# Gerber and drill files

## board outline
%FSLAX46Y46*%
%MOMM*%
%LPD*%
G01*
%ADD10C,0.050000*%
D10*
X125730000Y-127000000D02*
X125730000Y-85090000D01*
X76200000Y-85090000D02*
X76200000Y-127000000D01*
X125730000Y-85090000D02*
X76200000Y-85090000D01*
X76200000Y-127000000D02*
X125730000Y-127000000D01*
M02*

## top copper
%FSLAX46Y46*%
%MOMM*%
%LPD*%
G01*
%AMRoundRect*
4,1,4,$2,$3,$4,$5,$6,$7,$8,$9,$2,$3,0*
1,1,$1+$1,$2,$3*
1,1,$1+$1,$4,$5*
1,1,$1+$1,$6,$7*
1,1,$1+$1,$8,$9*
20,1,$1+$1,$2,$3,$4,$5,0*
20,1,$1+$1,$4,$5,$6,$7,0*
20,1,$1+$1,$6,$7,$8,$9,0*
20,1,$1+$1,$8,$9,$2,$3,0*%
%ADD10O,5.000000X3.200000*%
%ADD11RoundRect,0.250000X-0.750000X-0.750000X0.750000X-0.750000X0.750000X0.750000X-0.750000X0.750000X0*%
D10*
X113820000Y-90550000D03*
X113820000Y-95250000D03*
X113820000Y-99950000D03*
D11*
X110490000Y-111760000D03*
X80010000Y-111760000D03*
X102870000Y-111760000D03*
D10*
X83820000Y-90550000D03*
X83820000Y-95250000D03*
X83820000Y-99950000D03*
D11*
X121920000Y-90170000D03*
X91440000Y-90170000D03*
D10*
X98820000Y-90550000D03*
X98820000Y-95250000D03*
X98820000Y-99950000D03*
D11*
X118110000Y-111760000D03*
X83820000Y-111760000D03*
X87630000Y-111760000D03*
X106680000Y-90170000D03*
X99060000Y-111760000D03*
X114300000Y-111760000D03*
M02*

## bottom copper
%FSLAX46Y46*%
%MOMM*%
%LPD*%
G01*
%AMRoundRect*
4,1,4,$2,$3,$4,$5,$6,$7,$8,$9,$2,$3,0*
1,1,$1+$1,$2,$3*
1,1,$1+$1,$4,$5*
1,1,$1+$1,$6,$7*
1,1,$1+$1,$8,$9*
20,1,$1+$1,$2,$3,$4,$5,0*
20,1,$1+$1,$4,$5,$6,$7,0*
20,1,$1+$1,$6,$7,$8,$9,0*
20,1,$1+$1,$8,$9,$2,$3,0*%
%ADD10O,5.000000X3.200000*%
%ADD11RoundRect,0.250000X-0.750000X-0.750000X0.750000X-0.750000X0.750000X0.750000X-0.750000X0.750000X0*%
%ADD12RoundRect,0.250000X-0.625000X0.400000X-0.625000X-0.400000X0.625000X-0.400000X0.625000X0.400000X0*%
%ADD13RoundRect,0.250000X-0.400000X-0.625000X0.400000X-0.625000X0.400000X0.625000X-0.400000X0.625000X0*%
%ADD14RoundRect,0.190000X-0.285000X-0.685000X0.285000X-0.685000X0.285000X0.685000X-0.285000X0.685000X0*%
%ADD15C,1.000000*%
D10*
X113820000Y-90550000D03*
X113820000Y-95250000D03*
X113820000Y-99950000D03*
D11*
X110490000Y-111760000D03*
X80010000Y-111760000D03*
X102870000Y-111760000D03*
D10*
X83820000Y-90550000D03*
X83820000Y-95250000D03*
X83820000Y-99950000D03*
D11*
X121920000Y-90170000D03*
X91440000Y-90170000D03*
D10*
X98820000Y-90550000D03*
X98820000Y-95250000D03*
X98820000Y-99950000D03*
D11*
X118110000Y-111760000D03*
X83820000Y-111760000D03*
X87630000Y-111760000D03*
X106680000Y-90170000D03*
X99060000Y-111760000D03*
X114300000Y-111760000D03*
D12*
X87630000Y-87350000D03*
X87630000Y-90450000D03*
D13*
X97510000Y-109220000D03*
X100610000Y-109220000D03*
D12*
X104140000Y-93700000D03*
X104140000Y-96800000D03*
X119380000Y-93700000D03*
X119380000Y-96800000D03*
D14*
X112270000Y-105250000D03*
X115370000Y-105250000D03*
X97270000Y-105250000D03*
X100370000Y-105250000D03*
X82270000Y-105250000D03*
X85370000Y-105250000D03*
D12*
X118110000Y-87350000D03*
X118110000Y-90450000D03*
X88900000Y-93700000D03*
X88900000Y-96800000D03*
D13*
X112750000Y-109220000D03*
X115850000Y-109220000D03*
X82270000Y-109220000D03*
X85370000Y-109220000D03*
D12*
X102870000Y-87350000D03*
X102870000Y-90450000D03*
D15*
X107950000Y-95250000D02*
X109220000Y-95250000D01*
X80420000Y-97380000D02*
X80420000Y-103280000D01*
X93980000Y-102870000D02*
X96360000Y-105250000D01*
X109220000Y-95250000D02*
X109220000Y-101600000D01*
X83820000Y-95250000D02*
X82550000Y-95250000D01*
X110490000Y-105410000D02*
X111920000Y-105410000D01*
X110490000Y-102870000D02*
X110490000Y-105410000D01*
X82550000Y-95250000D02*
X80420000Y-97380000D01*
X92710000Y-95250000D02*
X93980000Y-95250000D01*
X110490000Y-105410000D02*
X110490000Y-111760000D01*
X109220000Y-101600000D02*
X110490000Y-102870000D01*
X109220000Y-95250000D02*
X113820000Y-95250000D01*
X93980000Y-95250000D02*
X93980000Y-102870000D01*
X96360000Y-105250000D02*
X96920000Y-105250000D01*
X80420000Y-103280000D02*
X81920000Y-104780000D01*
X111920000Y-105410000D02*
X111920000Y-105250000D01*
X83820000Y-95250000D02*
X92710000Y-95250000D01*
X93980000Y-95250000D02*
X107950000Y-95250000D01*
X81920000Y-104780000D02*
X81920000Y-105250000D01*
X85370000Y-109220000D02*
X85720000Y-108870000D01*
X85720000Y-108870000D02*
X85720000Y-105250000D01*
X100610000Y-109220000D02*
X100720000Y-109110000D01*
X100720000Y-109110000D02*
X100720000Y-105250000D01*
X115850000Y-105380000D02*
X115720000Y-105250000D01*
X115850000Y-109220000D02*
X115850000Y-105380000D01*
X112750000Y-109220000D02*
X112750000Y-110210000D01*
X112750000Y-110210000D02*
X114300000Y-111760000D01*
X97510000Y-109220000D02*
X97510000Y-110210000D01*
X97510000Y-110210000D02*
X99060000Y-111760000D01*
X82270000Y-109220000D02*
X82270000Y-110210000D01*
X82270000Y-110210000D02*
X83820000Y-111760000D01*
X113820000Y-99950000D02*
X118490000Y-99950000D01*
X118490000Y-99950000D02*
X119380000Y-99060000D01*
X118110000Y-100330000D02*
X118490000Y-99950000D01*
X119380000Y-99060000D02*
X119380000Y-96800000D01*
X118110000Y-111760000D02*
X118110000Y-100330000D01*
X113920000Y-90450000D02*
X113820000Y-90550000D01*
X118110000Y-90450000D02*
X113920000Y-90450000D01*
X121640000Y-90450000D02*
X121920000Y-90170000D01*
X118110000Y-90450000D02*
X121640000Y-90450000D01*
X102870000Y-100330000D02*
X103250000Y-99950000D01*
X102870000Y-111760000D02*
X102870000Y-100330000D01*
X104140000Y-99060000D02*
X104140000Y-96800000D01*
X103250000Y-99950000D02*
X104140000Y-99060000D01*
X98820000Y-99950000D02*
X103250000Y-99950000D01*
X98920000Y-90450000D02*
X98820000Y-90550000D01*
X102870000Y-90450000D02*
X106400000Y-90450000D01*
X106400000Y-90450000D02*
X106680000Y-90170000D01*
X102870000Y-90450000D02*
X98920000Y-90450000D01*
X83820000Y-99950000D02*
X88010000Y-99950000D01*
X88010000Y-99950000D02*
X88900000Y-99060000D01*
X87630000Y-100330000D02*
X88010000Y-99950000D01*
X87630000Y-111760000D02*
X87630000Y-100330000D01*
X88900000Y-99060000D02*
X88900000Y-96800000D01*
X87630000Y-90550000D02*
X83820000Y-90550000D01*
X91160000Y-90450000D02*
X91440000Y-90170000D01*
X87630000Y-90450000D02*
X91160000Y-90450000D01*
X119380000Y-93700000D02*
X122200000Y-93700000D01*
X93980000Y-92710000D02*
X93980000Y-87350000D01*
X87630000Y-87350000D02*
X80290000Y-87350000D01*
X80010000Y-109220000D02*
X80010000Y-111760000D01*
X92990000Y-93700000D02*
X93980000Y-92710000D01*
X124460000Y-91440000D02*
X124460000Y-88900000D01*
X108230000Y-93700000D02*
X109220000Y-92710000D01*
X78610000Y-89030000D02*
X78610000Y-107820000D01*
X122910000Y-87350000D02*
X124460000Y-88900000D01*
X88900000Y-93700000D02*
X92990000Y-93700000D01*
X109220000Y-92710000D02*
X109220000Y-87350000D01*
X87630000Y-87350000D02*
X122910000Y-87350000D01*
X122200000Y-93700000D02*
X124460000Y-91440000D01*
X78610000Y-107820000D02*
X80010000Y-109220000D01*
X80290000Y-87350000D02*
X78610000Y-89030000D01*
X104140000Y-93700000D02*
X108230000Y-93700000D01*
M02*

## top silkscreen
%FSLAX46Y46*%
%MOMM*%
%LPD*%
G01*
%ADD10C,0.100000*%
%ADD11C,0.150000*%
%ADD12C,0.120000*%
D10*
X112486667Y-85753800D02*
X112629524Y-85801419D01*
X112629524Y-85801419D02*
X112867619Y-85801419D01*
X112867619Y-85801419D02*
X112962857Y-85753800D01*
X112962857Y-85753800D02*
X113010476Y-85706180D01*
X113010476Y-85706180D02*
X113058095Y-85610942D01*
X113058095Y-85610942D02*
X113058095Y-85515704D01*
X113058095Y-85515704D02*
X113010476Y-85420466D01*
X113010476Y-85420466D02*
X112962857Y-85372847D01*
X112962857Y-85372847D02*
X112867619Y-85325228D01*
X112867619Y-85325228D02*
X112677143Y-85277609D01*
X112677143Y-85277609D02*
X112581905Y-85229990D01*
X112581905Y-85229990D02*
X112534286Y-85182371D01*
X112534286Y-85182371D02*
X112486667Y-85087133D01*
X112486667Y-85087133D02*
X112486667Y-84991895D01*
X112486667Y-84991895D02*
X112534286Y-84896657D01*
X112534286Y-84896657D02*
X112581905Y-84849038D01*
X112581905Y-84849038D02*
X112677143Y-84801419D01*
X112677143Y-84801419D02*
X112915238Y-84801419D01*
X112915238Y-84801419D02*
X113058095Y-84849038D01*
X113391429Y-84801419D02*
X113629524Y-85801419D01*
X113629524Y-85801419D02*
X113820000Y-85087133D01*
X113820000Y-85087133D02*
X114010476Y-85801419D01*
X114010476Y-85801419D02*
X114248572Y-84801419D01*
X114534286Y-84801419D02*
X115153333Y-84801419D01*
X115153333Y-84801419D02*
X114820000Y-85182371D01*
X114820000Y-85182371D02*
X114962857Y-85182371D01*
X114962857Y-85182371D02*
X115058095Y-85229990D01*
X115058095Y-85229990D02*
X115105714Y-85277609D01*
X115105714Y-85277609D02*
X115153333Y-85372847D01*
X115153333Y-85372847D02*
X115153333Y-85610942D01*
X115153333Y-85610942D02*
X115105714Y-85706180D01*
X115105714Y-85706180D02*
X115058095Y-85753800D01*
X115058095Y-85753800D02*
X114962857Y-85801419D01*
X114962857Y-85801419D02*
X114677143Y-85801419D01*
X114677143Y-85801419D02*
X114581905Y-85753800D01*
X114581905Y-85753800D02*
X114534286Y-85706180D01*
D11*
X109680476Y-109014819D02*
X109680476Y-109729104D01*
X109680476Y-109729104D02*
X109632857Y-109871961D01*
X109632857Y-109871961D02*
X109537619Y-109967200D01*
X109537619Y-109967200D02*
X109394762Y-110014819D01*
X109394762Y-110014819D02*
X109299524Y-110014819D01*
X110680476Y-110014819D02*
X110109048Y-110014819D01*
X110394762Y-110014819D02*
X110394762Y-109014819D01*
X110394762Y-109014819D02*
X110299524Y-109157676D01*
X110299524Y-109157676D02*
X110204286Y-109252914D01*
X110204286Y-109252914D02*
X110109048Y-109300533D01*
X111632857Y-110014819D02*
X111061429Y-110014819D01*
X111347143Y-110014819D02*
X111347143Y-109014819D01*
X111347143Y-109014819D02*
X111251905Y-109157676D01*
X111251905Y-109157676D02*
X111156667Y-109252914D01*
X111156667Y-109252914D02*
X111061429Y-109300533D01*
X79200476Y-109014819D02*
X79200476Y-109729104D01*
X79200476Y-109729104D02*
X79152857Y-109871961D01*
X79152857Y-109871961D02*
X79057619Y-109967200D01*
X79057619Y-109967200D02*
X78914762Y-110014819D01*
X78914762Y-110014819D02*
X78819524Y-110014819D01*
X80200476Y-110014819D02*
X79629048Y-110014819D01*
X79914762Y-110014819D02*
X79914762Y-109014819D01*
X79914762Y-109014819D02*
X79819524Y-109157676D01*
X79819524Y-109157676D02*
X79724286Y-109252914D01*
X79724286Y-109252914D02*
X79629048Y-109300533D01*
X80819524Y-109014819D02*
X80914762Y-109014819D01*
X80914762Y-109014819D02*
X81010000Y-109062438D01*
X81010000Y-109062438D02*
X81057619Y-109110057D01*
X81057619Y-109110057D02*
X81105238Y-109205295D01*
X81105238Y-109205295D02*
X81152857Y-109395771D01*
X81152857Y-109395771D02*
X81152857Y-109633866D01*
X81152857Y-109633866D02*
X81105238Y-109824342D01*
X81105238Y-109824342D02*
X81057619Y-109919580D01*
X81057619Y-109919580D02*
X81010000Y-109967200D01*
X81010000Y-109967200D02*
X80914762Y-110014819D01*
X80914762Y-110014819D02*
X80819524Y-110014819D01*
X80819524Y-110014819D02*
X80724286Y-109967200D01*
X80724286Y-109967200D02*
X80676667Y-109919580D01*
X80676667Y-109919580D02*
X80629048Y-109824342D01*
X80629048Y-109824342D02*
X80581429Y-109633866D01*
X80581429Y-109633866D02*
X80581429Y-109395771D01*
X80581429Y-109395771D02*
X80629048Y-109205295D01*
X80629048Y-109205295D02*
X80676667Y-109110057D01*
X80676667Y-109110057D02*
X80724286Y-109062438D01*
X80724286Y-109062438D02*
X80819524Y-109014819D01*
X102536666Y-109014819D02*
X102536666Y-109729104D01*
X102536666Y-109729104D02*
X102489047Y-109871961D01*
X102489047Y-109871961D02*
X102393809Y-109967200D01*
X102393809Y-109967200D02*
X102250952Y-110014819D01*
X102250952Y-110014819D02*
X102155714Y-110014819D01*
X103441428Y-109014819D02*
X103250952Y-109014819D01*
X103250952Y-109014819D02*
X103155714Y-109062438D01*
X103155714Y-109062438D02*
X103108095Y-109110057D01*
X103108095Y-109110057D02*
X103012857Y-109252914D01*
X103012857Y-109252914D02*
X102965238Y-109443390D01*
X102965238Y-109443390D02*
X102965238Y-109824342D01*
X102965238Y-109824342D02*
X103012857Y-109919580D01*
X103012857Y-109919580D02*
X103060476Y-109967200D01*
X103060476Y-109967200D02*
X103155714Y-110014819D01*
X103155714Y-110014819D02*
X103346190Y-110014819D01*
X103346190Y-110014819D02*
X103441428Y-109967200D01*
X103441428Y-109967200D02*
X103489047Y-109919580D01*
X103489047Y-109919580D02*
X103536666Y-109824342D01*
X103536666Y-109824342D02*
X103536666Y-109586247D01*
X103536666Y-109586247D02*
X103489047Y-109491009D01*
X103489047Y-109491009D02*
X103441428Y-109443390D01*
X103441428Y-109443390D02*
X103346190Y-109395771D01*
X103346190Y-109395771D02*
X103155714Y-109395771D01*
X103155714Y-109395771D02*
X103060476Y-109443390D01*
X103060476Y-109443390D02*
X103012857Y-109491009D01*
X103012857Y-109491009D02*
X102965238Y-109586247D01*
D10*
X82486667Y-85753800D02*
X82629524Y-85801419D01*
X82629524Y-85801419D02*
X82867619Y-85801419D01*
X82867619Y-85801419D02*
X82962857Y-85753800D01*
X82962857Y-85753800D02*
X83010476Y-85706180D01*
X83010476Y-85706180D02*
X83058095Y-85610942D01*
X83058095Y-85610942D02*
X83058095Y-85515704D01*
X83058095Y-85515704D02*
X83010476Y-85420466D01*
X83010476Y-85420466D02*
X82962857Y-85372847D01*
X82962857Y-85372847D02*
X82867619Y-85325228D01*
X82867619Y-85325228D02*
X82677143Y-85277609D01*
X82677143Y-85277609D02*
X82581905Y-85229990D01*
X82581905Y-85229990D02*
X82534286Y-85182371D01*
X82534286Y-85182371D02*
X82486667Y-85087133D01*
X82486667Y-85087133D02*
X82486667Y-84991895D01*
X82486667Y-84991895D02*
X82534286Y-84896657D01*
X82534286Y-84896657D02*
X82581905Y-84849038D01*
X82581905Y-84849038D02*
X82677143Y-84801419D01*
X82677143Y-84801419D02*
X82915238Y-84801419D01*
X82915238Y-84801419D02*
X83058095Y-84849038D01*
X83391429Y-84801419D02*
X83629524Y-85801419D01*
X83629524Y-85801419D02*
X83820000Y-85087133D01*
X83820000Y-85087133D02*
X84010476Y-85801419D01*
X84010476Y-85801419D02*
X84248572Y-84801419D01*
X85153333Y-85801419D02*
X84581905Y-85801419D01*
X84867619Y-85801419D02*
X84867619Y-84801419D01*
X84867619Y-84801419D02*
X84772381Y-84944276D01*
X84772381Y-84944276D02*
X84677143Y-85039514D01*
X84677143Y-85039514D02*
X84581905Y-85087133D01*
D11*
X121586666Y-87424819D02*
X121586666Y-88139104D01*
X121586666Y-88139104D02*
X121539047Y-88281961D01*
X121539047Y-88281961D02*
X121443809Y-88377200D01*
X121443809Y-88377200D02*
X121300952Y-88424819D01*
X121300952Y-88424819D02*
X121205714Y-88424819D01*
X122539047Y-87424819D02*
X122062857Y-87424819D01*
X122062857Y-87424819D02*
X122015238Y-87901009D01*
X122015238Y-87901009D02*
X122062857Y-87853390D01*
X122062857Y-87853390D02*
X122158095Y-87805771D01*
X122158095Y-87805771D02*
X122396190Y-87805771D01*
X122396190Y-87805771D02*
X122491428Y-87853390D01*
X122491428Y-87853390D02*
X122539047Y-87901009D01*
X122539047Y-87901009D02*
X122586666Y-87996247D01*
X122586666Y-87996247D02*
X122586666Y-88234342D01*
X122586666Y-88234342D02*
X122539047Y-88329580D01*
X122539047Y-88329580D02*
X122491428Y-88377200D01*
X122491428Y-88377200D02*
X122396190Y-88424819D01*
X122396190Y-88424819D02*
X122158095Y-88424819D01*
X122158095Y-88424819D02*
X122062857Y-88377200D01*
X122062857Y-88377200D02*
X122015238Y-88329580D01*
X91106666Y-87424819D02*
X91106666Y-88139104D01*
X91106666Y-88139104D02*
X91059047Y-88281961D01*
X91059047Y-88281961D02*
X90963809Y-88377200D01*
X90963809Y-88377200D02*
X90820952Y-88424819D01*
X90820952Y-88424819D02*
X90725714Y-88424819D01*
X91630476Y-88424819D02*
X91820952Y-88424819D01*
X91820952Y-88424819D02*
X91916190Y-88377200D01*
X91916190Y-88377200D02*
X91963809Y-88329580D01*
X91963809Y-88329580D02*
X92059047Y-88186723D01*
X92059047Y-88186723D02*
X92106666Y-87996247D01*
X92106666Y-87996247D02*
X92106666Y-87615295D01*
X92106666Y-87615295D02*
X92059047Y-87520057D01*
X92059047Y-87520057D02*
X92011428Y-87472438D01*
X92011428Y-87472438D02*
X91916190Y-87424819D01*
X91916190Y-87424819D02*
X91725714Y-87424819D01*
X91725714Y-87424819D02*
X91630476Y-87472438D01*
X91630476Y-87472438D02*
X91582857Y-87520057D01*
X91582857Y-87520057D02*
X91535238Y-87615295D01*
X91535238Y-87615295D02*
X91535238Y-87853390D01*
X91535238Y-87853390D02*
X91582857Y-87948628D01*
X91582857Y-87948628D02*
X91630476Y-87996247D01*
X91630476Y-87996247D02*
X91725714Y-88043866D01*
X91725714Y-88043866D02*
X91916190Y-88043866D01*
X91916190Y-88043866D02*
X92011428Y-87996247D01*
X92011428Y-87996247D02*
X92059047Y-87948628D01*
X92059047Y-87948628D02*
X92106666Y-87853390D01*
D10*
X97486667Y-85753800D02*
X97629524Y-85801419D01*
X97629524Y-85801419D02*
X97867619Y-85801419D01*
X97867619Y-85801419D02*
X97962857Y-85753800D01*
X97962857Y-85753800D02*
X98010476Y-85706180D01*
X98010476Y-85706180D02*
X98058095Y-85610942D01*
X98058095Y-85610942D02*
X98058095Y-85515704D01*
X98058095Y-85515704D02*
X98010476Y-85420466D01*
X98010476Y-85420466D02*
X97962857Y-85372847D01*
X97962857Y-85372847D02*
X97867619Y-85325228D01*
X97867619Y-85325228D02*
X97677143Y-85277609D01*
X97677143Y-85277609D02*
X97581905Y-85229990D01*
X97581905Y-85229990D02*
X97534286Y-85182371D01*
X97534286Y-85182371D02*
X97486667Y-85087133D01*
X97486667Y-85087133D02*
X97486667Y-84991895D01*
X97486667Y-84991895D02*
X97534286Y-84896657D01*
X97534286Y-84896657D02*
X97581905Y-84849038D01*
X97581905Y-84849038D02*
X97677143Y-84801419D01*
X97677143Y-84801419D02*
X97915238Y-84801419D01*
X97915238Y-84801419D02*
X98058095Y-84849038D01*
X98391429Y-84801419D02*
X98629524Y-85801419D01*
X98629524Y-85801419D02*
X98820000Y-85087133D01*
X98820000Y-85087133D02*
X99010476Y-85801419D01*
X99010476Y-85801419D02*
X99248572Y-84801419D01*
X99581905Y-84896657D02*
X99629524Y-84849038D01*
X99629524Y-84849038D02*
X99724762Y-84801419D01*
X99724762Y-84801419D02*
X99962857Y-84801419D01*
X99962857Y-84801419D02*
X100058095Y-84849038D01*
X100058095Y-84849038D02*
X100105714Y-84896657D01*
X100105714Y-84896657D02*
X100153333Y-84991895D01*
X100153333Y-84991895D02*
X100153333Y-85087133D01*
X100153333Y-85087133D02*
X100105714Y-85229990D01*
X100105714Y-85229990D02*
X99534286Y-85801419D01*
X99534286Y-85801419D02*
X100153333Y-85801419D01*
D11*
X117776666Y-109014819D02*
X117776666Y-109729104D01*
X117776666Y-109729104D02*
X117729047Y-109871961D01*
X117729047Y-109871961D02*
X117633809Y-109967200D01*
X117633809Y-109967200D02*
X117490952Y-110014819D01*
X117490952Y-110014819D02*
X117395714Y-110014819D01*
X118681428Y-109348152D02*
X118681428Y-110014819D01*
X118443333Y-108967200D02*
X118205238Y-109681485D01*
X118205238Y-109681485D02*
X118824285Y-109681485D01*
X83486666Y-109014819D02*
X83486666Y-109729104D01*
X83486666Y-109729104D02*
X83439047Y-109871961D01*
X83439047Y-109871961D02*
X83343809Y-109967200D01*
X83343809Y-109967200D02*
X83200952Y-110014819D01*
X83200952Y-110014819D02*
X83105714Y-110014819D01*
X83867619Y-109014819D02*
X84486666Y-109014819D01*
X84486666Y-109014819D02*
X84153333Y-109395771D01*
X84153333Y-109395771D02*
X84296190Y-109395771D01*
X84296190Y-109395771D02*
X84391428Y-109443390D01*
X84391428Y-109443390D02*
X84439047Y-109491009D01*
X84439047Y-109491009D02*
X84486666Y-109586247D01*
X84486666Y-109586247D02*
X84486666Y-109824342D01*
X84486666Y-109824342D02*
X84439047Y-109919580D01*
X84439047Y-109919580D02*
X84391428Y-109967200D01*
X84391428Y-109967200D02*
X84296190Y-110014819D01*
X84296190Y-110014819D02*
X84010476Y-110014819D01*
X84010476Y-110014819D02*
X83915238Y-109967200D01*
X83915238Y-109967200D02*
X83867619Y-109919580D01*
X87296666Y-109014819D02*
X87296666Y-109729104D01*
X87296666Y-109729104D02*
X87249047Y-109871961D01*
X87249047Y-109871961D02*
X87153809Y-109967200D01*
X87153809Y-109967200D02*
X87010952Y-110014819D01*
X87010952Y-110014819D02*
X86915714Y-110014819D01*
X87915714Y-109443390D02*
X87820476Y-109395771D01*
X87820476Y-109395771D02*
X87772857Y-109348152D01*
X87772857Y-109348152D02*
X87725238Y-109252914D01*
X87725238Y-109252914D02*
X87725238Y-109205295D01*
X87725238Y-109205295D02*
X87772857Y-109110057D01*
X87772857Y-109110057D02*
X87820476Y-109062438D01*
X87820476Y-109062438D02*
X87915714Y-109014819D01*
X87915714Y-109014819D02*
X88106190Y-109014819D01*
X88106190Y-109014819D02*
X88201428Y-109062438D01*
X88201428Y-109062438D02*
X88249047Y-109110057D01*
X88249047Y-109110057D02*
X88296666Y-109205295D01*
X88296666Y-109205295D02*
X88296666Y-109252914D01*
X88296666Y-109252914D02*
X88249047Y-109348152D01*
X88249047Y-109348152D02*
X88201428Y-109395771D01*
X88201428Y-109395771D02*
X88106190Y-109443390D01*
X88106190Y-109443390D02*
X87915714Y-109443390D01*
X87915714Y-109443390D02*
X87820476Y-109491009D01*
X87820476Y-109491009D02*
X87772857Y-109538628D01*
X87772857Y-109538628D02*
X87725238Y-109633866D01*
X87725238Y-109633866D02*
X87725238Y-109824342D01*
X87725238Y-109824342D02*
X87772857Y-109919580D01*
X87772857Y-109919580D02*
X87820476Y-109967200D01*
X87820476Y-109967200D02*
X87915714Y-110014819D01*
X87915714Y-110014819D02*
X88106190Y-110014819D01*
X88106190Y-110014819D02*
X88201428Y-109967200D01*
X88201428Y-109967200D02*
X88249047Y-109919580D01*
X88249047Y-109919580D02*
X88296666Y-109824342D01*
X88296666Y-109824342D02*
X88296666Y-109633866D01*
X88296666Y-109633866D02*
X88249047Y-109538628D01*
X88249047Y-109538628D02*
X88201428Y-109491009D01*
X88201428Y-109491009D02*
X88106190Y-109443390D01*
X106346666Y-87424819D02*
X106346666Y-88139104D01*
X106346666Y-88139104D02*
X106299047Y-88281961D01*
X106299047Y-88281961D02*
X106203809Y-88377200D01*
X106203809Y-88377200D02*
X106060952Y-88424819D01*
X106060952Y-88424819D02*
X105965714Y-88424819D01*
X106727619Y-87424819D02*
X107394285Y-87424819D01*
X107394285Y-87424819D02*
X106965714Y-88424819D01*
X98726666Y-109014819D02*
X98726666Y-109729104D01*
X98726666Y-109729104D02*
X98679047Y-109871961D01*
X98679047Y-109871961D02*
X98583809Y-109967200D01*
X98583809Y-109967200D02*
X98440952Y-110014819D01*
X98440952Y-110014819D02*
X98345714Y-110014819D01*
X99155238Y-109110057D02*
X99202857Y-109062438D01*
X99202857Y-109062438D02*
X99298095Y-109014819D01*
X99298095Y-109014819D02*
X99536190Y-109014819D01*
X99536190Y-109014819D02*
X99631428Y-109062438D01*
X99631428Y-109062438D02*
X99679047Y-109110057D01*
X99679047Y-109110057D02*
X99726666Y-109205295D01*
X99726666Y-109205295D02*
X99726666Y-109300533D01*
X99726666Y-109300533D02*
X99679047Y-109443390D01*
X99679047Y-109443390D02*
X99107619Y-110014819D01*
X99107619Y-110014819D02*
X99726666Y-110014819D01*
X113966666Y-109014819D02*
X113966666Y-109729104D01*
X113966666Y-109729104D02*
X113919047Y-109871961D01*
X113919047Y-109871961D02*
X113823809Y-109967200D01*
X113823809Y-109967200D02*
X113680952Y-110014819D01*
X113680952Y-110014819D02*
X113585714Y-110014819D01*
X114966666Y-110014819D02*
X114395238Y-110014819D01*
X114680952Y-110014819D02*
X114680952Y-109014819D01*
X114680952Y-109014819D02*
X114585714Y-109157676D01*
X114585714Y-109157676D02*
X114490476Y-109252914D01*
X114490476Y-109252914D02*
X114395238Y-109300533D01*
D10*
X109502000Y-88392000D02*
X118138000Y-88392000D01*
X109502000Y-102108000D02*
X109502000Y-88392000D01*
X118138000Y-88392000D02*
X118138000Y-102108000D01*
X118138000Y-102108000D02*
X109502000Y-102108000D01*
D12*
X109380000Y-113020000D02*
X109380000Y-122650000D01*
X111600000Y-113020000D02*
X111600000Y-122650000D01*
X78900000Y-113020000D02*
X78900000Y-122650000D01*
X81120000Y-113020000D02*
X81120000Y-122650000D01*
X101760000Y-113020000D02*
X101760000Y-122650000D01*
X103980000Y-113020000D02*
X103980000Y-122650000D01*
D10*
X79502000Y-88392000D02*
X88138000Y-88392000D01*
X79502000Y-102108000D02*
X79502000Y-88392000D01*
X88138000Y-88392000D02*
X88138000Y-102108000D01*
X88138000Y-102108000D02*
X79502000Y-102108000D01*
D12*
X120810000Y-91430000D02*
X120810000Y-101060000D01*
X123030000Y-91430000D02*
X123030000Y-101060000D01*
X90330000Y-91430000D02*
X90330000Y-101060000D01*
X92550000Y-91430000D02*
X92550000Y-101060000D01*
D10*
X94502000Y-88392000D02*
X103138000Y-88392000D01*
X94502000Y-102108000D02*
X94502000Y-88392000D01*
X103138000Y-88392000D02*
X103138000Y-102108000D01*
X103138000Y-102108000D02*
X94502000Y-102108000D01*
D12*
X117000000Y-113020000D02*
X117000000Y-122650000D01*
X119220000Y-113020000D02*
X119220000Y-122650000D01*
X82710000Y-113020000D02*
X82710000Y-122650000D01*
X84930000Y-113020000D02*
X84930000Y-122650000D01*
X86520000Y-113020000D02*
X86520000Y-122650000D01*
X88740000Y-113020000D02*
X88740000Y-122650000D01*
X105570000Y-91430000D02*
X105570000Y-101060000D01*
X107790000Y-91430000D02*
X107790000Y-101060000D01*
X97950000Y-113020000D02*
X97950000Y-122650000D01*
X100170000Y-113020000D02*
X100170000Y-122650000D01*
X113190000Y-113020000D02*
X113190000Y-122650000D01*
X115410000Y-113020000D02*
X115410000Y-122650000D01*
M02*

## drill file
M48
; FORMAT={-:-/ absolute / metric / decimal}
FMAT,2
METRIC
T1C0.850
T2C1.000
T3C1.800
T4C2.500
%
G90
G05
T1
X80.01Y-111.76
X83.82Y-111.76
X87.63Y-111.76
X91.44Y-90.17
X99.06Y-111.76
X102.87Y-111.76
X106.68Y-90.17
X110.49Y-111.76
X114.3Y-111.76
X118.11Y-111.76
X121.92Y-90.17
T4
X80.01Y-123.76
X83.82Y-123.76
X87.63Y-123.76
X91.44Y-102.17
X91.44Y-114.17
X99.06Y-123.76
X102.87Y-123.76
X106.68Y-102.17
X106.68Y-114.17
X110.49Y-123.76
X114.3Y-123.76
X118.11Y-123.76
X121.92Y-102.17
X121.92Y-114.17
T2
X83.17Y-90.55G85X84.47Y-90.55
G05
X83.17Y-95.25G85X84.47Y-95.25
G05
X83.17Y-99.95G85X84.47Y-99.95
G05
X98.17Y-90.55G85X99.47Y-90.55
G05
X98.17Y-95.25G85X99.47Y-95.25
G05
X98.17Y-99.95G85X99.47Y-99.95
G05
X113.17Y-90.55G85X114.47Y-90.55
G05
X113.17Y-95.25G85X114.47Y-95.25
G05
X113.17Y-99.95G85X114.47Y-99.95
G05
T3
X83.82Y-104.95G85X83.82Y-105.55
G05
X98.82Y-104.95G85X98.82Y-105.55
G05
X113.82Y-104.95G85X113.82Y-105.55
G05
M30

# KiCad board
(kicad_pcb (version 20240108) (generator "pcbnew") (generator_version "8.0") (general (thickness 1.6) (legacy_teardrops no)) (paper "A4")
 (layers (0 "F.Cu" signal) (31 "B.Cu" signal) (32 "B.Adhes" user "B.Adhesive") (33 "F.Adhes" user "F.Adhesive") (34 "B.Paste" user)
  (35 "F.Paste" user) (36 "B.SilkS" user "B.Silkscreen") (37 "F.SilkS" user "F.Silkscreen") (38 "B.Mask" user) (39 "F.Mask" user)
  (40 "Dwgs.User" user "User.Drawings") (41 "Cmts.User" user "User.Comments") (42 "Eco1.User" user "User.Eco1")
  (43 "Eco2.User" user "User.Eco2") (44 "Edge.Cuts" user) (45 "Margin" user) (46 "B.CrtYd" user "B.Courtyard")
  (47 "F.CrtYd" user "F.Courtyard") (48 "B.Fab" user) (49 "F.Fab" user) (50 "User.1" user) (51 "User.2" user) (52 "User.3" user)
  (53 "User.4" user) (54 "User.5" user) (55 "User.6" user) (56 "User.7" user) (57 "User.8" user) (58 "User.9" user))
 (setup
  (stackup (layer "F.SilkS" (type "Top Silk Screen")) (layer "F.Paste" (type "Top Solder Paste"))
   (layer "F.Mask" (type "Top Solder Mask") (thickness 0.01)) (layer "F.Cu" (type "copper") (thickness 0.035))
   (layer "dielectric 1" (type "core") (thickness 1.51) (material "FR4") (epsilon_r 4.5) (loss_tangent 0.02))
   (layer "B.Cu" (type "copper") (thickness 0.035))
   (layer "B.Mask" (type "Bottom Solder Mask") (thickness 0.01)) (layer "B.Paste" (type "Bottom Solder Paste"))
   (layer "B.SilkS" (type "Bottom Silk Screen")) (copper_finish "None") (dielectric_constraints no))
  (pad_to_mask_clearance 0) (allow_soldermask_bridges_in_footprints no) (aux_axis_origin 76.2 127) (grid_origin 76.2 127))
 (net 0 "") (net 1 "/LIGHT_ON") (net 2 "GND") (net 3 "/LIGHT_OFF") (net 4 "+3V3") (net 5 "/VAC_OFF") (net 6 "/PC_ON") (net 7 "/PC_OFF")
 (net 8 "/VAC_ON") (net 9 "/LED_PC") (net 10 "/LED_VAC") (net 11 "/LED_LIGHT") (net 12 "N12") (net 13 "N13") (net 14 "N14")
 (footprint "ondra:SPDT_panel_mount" (layer "F.Cu") (at 113.82 95.25)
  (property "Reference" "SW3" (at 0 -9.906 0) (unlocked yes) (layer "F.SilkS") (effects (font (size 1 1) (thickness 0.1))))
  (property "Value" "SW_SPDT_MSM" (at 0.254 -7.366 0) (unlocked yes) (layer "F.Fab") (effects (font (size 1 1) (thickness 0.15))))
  (fp_line (start -4.318 -6.858) (end 4.318 -6.858) (stroke (width 0.1) (type default)) (layer "F.SilkS"))
  (fp_line (start -4.318 6.858) (end -4.318 -6.858) (stroke (width 0.1) (type default)) (layer "F.SilkS"))
  (fp_line (start 4.318 -6.858) (end 4.318 6.858) (stroke (width 0.1) (type default)) (layer "F.SilkS"))
  (fp_line (start 4.318 6.858) (end -4.318 6.858) (stroke (width 0.1) (type default)) (layer "F.SilkS"))
  (pad "1" thru_hole oval (at 0 -4.7) (size 5 3.2) (drill oval 2.3 1) (layers "*.Cu" "*.Mask") (remove_unused_layers no) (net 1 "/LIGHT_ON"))
  (pad "2" thru_hole oval (at 0 0) (size 5 3.2) (drill oval 2.3 1) (layers "*.Cu" "*.Mask") (remove_unused_layers no) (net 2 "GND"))
  (pad "3" thru_hole oval (at 0 4.7) (size 5 3.2) (drill oval 2.3 1) (layers "*.Cu" "*.Mask") (remove_unused_layers no) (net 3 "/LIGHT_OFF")))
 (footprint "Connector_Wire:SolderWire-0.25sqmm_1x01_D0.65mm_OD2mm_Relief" (layer "F.Cu") (at 110.49 111.76)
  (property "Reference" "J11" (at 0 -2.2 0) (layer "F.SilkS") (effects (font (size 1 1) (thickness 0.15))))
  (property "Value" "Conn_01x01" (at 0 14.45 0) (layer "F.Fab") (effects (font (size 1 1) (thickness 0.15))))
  (fp_line (start -1.11 1.26) (end -1.11 10.89) (stroke (width 0.12) (type solid)) (layer "F.SilkS"))
  (fp_line (start 1.11 1.26) (end 1.11 10.89) (stroke (width 0.12) (type solid)) (layer "F.SilkS"))
  (pad "" np_thru_hole circle (at 0 12) (size 2.5 2.5) (drill 2.5) (layers "*.Cu" "*.Mask"))
  (pad "1" thru_hole roundrect (at 0 0) (size 2 2) (drill 0.85) (layers "*.Cu" "*.Mask") (remove_unused_layers no) (roundrect_rratio 0.125)
   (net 2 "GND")))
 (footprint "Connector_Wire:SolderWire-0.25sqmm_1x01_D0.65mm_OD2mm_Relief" (layer "F.Cu") (at 80.01 111.76)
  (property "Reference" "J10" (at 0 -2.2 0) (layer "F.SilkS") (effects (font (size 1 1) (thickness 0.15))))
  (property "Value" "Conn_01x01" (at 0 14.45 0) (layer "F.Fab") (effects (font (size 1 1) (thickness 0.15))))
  (fp_line (start -1.11 1.26) (end -1.11 10.89) (stroke (width 0.12) (type solid)) (layer "F.SilkS"))
  (fp_line (start 1.11 1.26) (end 1.11 10.89) (stroke (width 0.12) (type solid)) (layer "F.SilkS"))
  (pad "" np_thru_hole circle (at 0 12) (size 2.5 2.5) (drill 2.5) (layers "*.Cu" "*.Mask"))
  (pad "1" thru_hole roundrect (at 0 0) (size 2 2) (drill 0.85) (layers "*.Cu" "*.Mask") (remove_unused_layers no) (roundrect_rratio 0.125)
   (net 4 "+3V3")))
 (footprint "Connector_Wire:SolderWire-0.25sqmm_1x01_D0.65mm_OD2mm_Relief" (layer "F.Cu") (at 102.87 111.76)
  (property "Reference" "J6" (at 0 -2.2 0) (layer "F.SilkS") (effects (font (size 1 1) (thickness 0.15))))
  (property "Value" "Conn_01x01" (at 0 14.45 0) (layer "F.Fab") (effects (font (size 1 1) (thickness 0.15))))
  (fp_line (start -1.11 1.26) (end -1.11 10.89) (stroke (width 0.12) (type solid)) (layer "F.SilkS"))
  (fp_line (start 1.11 1.26) (end 1.11 10.89) (stroke (width 0.12) (type solid)) (layer "F.SilkS"))
  (pad "" np_thru_hole circle (at 0 12) (size 2.5 2.5) (drill 2.5) (layers "*.Cu" "*.Mask"))
  (pad "1" thru_hole roundrect (at 0 0) (size 2 2) (drill 0.85) (layers "*.Cu" "*.Mask") (remove_unused_layers no) (roundrect_rratio 0.125)
   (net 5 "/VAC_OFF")))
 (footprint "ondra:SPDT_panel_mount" (layer "F.Cu") (at 83.82 95.25)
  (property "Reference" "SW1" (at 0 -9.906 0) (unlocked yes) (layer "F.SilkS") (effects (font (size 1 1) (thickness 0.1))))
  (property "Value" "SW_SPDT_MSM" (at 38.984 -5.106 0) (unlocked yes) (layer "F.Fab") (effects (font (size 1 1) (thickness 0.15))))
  (fp_line (start -4.318 -6.858) (end 4.318 -6.858) (stroke (width 0.1) (type default)) (layer "F.SilkS"))
  (fp_line (start -4.318 6.858) (end -4.318 -6.858) (stroke (width 0.1) (type default)) (layer "F.SilkS"))
  (fp_line (start 4.318 -6.858) (end 4.318 6.858) (stroke (width 0.1) (type default)) (layer "F.SilkS"))
  (fp_line (start 4.318 6.858) (end -4.318 6.858) (stroke (width 0.1) (type default)) (layer "F.SilkS"))
  (pad "1" thru_hole oval (at 0 -4.7) (size 5 3.2) (drill oval 2.3 1) (layers "*.Cu" "*.Mask") (remove_unused_layers no) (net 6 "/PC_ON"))
  (pad "2" thru_hole oval (at 0 0) (size 5 3.2) (drill oval 2.3 1) (layers "*.Cu" "*.Mask") (remove_unused_layers no) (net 2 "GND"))
  (pad "3" thru_hole oval (at 0 4.7) (size 5 3.2) (drill oval 2.3 1) (layers "*.Cu" "*.Mask") (remove_unused_layers no) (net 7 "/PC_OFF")))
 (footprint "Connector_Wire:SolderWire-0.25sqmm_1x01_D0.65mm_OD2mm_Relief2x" (layer "F.Cu") (at 121.92 90.17)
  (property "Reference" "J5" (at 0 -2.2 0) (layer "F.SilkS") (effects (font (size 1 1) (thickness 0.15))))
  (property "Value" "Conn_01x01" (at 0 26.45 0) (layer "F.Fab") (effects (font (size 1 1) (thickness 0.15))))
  (fp_line (start -1.11 1.26) (end -1.11 10.89) (stroke (width 0.12) (type solid)) (layer "F.SilkS"))
  (fp_line (start 1.11 1.26) (end 1.11 10.89) (stroke (width 0.12) (type solid)) (layer "F.SilkS"))
  (pad "" np_thru_hole circle (at 0 12) (size 2.5 2.5) (drill 2.5) (layers "*.Cu" "*.Mask"))
  (pad "" np_thru_hole circle (at 0 24) (size 2.5 2.5) (drill 2.5) (layers "*.Cu" "*.Mask"))
  (pad "1" thru_hole roundrect (at 0 0) (size 2 2) (drill 0.85) (layers "*.Cu" "*.Mask") (remove_unused_layers no) (roundrect_rratio 0.125)
   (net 1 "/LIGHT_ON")))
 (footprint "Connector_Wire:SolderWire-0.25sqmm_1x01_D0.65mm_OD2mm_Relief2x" (layer "F.Cu") (at 91.44 90.17)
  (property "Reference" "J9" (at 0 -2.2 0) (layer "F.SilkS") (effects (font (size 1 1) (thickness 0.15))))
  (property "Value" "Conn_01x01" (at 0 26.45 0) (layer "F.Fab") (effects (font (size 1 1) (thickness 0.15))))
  (fp_line (start -1.11 1.26) (end -1.11 10.89) (stroke (width 0.12) (type solid)) (layer "F.SilkS"))
  (fp_line (start 1.11 1.26) (end 1.11 10.89) (stroke (width 0.12) (type solid)) (layer "F.SilkS"))
  (pad "" np_thru_hole circle (at 0 12) (size 2.5 2.5) (drill 2.5) (layers "*.Cu" "*.Mask"))
  (pad "" np_thru_hole circle (at 0 24) (size 2.5 2.5) (drill 2.5) (layers "*.Cu" "*.Mask"))
  (pad "1" thru_hole roundrect (at 0 0) (size 2 2) (drill 0.85) (layers "*.Cu" "*.Mask") (remove_unused_layers no) (roundrect_rratio 0.125)
   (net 6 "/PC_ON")))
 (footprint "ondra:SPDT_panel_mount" (layer "F.Cu") (at 98.82 95.25)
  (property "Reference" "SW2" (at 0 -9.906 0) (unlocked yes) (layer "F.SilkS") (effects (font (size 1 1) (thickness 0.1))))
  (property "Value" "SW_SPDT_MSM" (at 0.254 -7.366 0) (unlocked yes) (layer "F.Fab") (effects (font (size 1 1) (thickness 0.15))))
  (fp_line (start -4.318 -6.858) (end 4.318 -6.858) (stroke (width 0.1) (type default)) (layer "F.SilkS"))
  (fp_line (start -4.318 6.858) (end -4.318 -6.858) (stroke (width 0.1) (type default)) (layer "F.SilkS"))
  (fp_line (start 4.318 -6.858) (end 4.318 6.858) (stroke (width 0.1) (type default)) (layer "F.SilkS"))
  (fp_line (start 4.318 6.858) (end -4.318 6.858) (stroke (width 0.1) (type default)) (layer "F.SilkS"))
  (pad "1" thru_hole oval (at 0 -4.7) (size 5 3.2) (drill oval 2.3 1) (layers "*.Cu" "*.Mask") (remove_unused_layers no) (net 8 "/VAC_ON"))
  (pad "2" thru_hole oval (at 0 0) (size 5 3.2) (drill oval 2.3 1) (layers "*.Cu" "*.Mask") (remove_unused_layers no) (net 2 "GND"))
  (pad "3" thru_hole oval (at 0 4.7) (size 5 3.2) (drill oval 2.3 1) (layers "*.Cu" "*.Mask") (remove_unused_layers no) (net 5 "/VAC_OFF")))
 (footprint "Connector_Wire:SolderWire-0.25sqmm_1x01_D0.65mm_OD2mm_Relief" (layer "F.Cu") (at 118.11 111.76)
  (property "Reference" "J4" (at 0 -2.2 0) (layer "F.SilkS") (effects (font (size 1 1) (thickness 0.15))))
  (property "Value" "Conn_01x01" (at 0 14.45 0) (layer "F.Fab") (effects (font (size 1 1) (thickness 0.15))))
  (fp_line (start -1.11 1.26) (end -1.11 10.89) (stroke (width 0.12) (type solid)) (layer "F.SilkS"))
  (fp_line (start 1.11 1.26) (end 1.11 10.89) (stroke (width 0.12) (type solid)) (layer "F.SilkS"))
  (pad "" np_thru_hole circle (at 0 12) (size 2.5 2.5) (drill 2.5) (layers "*.Cu" "*.Mask"))
  (pad "1" thru_hole roundrect (at 0 0) (size 2 2) (drill 0.85) (layers "*.Cu" "*.Mask") (remove_unused_layers no) (roundrect_rratio 0.125)
   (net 3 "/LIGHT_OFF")))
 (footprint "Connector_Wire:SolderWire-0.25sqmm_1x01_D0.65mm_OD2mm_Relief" (layer "F.Cu") (at 83.82 111.76)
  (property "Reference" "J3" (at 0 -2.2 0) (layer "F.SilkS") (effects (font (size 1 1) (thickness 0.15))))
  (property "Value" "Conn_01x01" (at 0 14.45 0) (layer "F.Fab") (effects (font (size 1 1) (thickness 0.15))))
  (fp_line (start -1.11 1.26) (end -1.11 10.89) (stroke (width 0.12) (type solid)) (layer "F.SilkS"))
  (fp_line (start 1.11 1.26) (end 1.11 10.89) (stroke (width 0.12) (type solid)) (layer "F.SilkS"))
  (pad "" np_thru_hole circle (at 0 12) (size 2.5 2.5) (drill 2.5) (layers "*.Cu" "*.Mask"))
  (pad "1" thru_hole roundrect (at 0 0) (size 2 2) (drill 0.85) (layers "*.Cu" "*.Mask") (remove_unused_layers no) (roundrect_rratio 0.125)
   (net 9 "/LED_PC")))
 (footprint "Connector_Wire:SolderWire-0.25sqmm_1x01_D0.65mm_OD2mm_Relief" (layer "F.Cu") (at 87.63 111.76)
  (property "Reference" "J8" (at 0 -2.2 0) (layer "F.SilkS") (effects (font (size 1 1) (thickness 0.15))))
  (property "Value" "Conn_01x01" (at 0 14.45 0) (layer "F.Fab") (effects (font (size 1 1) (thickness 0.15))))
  (fp_line (start -1.11 1.26) (end -1.11 10.89) (stroke (width 0.12) (type solid)) (layer "F.SilkS"))
  (fp_line (start 1.11 1.26) (end 1.11 10.89) (stroke (width 0.12) (type solid)) (layer "F.SilkS"))
  (pad "" np_thru_hole circle (at 0 12) (size 2.5 2.5) (drill 2.5) (layers "*.Cu" "*.Mask"))
  (pad "1" thru_hole roundrect (at 0 0) (size 2 2) (drill 0.85) (layers "*.Cu" "*.Mask") (remove_unused_layers no) (roundrect_rratio 0.125)
   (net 7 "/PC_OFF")))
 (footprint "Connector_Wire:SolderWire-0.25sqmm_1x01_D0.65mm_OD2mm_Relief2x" (layer "F.Cu") (at 106.68 90.17)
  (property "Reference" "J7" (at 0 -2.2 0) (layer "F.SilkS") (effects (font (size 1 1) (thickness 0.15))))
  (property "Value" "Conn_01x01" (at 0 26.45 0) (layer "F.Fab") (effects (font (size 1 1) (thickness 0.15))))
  (fp_line (start -1.11 1.26) (end -1.11 10.89) (stroke (width 0.12) (type solid)) (layer "F.SilkS"))
  (fp_line (start 1.11 1.26) (end 1.11 10.89) (stroke (width 0.12) (type solid)) (layer "F.SilkS"))
  (pad "" np_thru_hole circle (at 0 12) (size 2.5 2.5) (drill 2.5) (layers "*.Cu" "*.Mask"))
  (pad "" np_thru_hole circle (at 0 24) (size 2.5 2.5) (drill 2.5) (layers "*.Cu" "*.Mask"))
  (pad "1" thru_hole roundrect (at 0 0) (size 2 2) (drill 0.85) (layers "*.Cu" "*.Mask") (remove_unused_layers no) (roundrect_rratio 0.125)
   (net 8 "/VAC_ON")))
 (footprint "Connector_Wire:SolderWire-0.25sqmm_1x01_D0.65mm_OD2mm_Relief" (layer "F.Cu") (at 99.06 111.76)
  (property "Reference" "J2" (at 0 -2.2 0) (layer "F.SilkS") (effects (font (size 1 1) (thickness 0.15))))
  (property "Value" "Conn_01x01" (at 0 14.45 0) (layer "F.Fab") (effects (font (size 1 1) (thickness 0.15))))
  (fp_line (start -1.11 1.26) (end -1.11 10.89) (stroke (width 0.12) (type solid)) (layer "F.SilkS"))
  (fp_line (start 1.11 1.26) (end 1.11 10.89) (stroke (width 0.12) (type solid)) (layer "F.SilkS"))
  (pad "" np_thru_hole circle (at 0 12) (size 2.5 2.5) (drill 2.5) (layers "*.Cu" "*.Mask"))
  (pad "1" thru_hole roundrect (at 0 0) (size 2 2) (drill 0.85) (layers "*.Cu" "*.Mask") (remove_unused_layers no) (roundrect_rratio 0.125)
   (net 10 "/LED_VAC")))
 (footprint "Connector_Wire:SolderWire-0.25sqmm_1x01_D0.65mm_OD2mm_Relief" (layer "F.Cu") (at 114.3 111.76)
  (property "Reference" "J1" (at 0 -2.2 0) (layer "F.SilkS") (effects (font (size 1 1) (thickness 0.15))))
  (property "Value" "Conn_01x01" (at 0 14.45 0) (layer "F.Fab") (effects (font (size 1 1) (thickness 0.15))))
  (fp_line (start -1.11 1.26) (end -1.11 10.89) (stroke (width 0.12) (type solid)) (layer "F.SilkS"))
  (fp_line (start 1.11 1.26) (end 1.11 10.89) (stroke (width 0.12) (type solid)) (layer "F.SilkS"))
  (pad "" np_thru_hole circle (at 0 12) (size 2.5 2.5) (drill 2.5) (layers "*.Cu" "*.Mask"))
  (pad "1" thru_hole roundrect (at 0 0) (size 2 2) (drill 0.85) (layers "*.Cu" "*.Mask") (remove_unused_layers no) (roundrect_rratio 0.125)
   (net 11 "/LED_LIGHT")))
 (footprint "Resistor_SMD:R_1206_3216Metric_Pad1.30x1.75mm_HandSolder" (layer "B.Cu") (at 87.63 88.9 -90)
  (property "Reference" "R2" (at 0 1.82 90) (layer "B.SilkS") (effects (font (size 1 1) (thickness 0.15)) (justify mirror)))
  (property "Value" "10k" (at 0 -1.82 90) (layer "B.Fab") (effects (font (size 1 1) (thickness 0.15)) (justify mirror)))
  (pad "1" smd roundrect (at -1.55 0 270) (size 1.3 1.75) (layers "B.Cu" "B.Paste" "B.Mask") (roundrect_rratio 0.1923076923) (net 4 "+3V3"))
  (pad "2" smd roundrect (at 1.55 0 270) (size 1.3 1.75) (layers "B.Cu" "B.Paste" "B.Mask") (roundrect_rratio 0.1923076923) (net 6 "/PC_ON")))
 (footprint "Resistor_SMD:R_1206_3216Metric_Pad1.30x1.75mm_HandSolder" (layer "B.Cu") (at 99.06 109.22)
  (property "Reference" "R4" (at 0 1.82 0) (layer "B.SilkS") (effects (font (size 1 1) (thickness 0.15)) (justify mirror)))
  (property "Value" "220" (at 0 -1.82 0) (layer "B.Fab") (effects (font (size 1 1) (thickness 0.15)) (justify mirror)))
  (pad "1" smd roundrect (at -1.55 0) (size 1.3 1.75) (layers "B.Cu" "B.Paste" "B.Mask") (roundrect_rratio 0.1923076923) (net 10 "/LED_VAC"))
  (pad "2" smd roundrect (at 1.55 0) (size 1.3 1.75) (layers "B.Cu" "B.Paste" "B.Mask") (roundrect_rratio 0.1923076923) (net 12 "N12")))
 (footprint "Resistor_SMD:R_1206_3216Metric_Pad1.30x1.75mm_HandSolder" (layer "B.Cu") (at 104.14 95.25 -90)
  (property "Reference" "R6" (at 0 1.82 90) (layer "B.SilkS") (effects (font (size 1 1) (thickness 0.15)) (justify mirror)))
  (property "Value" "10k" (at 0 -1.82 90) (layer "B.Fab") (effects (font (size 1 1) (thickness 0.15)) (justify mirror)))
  (pad "1" smd roundrect (at -1.55 0 270) (size 1.3 1.75) (layers "B.Cu" "B.Paste" "B.Mask") (roundrect_rratio 0.1923076923) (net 4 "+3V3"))
  (pad "2" smd roundrect (at 1.55 0 270) (size 1.3 1.75) (layers "B.Cu" "B.Paste" "B.Mask") (roundrect_rratio 0.1923076923)
   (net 5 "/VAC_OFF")))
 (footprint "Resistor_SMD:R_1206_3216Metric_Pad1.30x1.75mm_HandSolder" (layer "B.Cu") (at 119.38 95.25 -90)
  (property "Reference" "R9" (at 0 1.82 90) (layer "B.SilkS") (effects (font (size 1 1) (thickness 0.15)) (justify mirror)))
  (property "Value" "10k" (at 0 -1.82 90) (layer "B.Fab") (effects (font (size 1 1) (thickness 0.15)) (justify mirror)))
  (pad "1" smd roundrect (at -1.55 0 270) (size 1.3 1.75) (layers "B.Cu" "B.Paste" "B.Mask") (roundrect_rratio 0.1923076923) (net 4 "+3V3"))
  (pad "2" smd roundrect (at 1.55 0 270) (size 1.3 1.75) (layers "B.Cu" "B.Paste" "B.Mask") (roundrect_rratio 0.1923076923)
   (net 3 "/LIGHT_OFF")))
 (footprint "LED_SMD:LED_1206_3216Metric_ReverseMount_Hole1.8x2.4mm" (layer "B.Cu") (at 113.82 105.25)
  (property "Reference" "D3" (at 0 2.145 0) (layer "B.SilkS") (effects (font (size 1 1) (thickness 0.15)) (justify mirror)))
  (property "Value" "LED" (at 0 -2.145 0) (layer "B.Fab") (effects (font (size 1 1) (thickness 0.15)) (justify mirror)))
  (pad "" np_thru_hole oval (at 0 0) (size 1.8 2.4) (drill oval 1.8 2.4) (layers "*.Cu" "*.Mask"))
  (pad "1" smd roundrect (at -1.55 0) (size 0.95 1.75) (layers "B.Cu" "B.Paste" "B.Mask") (roundrect_rratio 0.2) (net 2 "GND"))
  (pad "2" smd roundrect (at 1.55 0) (size 0.95 1.75) (layers "B.Cu" "B.Paste" "B.Mask") (roundrect_rratio 0.2) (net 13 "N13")))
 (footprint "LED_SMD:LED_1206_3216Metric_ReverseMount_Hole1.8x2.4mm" (layer "B.Cu") (at 98.82 105.25)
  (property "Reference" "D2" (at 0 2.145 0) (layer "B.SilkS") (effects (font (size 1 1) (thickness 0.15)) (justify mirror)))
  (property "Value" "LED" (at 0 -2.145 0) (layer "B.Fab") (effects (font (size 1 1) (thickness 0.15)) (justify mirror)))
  (pad "" np_thru_hole oval (at 0 0) (size 1.8 2.4) (drill oval 1.8 2.4) (layers "*.Cu" "*.Mask"))
  (pad "1" smd roundrect (at -1.55 0) (size 0.95 1.75) (layers "B.Cu" "B.Paste" "B.Mask") (roundrect_rratio 0.2) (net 2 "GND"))
  (pad "2" smd roundrect (at 1.55 0) (size 0.95 1.75) (layers "B.Cu" "B.Paste" "B.Mask") (roundrect_rratio 0.2) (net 12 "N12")))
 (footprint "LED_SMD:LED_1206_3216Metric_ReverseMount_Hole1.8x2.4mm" (layer "B.Cu") (at 83.82 105.25)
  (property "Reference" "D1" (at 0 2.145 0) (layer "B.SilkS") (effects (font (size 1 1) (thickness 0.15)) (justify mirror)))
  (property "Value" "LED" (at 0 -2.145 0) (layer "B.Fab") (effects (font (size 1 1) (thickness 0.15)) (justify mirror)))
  (pad "" np_thru_hole oval (at 0 0) (size 1.8 2.4) (drill oval 1.8 2.4) (layers "*.Cu" "*.Mask"))
  (pad "1" smd roundrect (at -1.55 0) (size 0.95 1.75) (layers "B.Cu" "B.Paste" "B.Mask") (roundrect_rratio 0.2) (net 2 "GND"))
  (pad "2" smd roundrect (at 1.55 0) (size 0.95 1.75) (layers "B.Cu" "B.Paste" "B.Mask") (roundrect_rratio 0.2) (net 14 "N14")))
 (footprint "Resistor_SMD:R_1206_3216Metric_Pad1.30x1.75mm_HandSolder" (layer "B.Cu") (at 118.11 88.9 -90)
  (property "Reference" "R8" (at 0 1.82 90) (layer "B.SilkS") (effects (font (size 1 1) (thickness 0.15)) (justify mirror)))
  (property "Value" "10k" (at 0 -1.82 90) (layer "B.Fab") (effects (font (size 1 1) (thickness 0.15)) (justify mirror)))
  (pad "1" smd roundrect (at -1.55 0 270) (size 1.3 1.75) (layers "B.Cu" "B.Paste" "B.Mask") (roundrect_rratio 0.1923076923) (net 4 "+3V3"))
  (pad "2" smd roundrect (at 1.55 0 270) (size 1.3 1.75) (layers "B.Cu" "B.Paste" "B.Mask") (roundrect_rratio 0.1923076923)
   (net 1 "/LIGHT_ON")))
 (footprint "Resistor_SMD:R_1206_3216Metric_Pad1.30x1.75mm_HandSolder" (layer "B.Cu") (at 88.9 95.25 -90)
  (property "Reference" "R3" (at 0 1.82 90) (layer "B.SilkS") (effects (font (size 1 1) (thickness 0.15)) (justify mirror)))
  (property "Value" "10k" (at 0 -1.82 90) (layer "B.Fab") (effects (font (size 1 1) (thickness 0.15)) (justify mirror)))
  (pad "1" smd roundrect (at -1.55 0 270) (size 1.3 1.75) (layers "B.Cu" "B.Paste" "B.Mask") (roundrect_rratio 0.1923076923) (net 4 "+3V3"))
  (pad "2" smd roundrect (at 1.55 0 270) (size 1.3 1.75) (layers "B.Cu" "B.Paste" "B.Mask") (roundrect_rratio 0.1923076923)
   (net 7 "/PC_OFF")))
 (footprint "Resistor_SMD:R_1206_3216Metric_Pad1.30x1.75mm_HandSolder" (layer "B.Cu") (at 114.3 109.22)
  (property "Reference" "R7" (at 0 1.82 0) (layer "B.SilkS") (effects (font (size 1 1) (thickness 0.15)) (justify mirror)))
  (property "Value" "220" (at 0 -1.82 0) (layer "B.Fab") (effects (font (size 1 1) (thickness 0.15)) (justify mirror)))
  (pad "1" smd roundrect (at -1.55 0) (size 1.3 1.75) (layers "B.Cu" "B.Paste" "B.Mask") (roundrect_rratio 0.1923076923)
   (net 11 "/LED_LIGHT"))
  (pad "2" smd roundrect (at 1.55 0) (size 1.3 1.75) (layers "B.Cu" "B.Paste" "B.Mask") (roundrect_rratio 0.1923076923) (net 13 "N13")))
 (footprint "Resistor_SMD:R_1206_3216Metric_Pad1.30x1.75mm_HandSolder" (layer "B.Cu") (at 83.82 109.22)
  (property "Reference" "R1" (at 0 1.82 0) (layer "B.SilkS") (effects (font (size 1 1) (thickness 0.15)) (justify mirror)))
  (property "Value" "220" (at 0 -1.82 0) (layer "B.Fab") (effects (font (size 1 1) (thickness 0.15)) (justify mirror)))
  (pad "1" smd roundrect (at -1.55 0) (size 1.3 1.75) (layers "B.Cu" "B.Paste" "B.Mask") (roundrect_rratio 0.1923076923) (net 9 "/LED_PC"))
  (pad "2" smd roundrect (at 1.55 0) (size 1.3 1.75) (layers "B.Cu" "B.Paste" "B.Mask") (roundrect_rratio 0.1923076923) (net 14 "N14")))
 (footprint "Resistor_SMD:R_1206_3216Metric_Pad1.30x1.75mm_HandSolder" (layer "B.Cu") (at 102.87 88.9 -90)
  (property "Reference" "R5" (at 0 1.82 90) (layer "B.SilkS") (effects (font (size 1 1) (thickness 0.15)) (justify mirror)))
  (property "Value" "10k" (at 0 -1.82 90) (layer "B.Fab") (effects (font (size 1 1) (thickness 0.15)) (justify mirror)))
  (pad "1" smd roundrect (at -1.55 0 270) (size 1.3 1.75) (layers "B.Cu" "B.Paste" "B.Mask") (roundrect_rratio 0.1923076923) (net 4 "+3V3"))
  (pad "2" smd roundrect (at 1.55 0 270) (size 1.3 1.75) (layers "B.Cu" "B.Paste" "B.Mask") (roundrect_rratio 0.1923076923)
   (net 8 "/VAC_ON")))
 (gr_line (start 125.73 127) (end 125.73 85.09) (stroke (width 0.05) (type default)) (layer "Edge.Cuts"))
 (gr_line (start 76.2 85.09) (end 76.2 127) (stroke (width 0.05) (type default)) (layer "Edge.Cuts"))
 (gr_line (start 125.73 85.09) (end 76.2 85.09) (stroke (width 0.05) (type default)) (layer "Edge.Cuts"))
 (gr_line (start 76.2 127) (end 125.73 127) (stroke (width 0.05) (type default)) (layer "Edge.Cuts"))
 (segment (start 107.95 95.25) (end 109.22 95.25) (width 1) (layer "B.Cu") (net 2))
 (segment (start 80.42 97.38) (end 80.42 103.28) (width 1) (layer "B.Cu") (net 2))
 (segment (start 93.98 102.87) (end 96.36 105.25) (width 1) (layer "B.Cu") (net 2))
 (segment (start 109.22 95.25) (end 109.22 101.6) (width 1) (layer "B.Cu") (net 2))
 (segment (start 83.82 95.25) (end 82.55 95.25) (width 1) (layer "B.Cu") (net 2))
 (segment (start 110.49 105.41) (end 111.92 105.41) (width 1) (layer "B.Cu") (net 2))
 (segment (start 110.49 102.87) (end 110.49 105.41) (width 1) (layer "B.Cu") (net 2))
 (segment (start 82.55 95.25) (end 80.42 97.38) (width 1) (layer "B.Cu") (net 2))
 (segment (start 92.71 95.25) (end 93.98 95.25) (width 1) (layer "B.Cu") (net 2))
 (segment (start 110.49 105.41) (end 110.49 111.76) (width 1) (layer "B.Cu") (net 2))
 (segment (start 109.22 101.6) (end 110.49 102.87) (width 1) (layer "B.Cu") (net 2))
 (segment (start 109.22 95.25) (end 113.82 95.25) (width 1) (layer "B.Cu") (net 2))
 (segment (start 93.98 95.25) (end 93.98 102.87) (width 1) (layer "B.Cu") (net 2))
 (segment (start 96.36 105.25) (end 96.92 105.25) (width 1) (layer "B.Cu") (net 2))
 (segment (start 80.42 103.28) (end 81.92 104.78) (width 1) (layer "B.Cu") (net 2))
 (segment (start 111.92 105.41) (end 111.92 105.25) (width 1) (layer "B.Cu") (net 2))
 (segment (start 83.82 95.25) (end 92.71 95.25) (width 1) (layer "B.Cu") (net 2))
 (segment (start 93.98 95.25) (end 107.95 95.25) (width 1) (layer "B.Cu") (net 2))
 (segment (start 81.92 104.78) (end 81.92 105.25) (width 1) (layer "B.Cu") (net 2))
 (segment (start 85.37 109.22) (end 85.72 108.87) (width 1) (layer "B.Cu") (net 14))
 (segment (start 85.72 108.87) (end 85.72 105.25) (width 1) (layer "B.Cu") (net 14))
 (segment (start 100.61 109.22) (end 100.72 109.11) (width 1) (layer "B.Cu") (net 12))
 (segment (start 100.72 109.11) (end 100.72 105.25) (width 1) (layer "B.Cu") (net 12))
 (segment (start 115.85 105.38) (end 115.72 105.25) (width 1) (layer "B.Cu") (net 13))
 (segment (start 115.85 109.22) (end 115.85 105.38) (width 1) (layer "B.Cu") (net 13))
 (segment (start 112.75 109.22) (end 112.75 110.21) (width 1) (layer "B.Cu") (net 11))
 (segment (start 112.75 110.21) (end 114.3 111.76) (width 1) (layer "B.Cu") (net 11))
 (segment (start 97.51 109.22) (end 97.51 110.21) (width 1) (layer "B.Cu") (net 10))
 (segment (start 97.51 110.21) (end 99.06 111.76) (width 1) (layer "B.Cu") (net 10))
 (segment (start 82.27 109.22) (end 82.27 110.21) (width 1) (layer "B.Cu") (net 9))
 (segment (start 82.27 110.21) (end 83.82 111.76) (width 1) (layer "B.Cu") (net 9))
 (segment (start 113.82 99.95) (end 118.49 99.95) (width 1) (layer "B.Cu") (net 3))
 (segment (start 118.49 99.95) (end 119.38 99.06) (width 1) (layer "B.Cu") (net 3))
 (segment (start 118.11 100.33) (end 118.49 99.95) (width 1) (layer "B.Cu") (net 3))
 (segment (start 119.38 99.06) (end 119.38 96.8) (width 1) (layer "B.Cu") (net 3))
 (segment (start 118.11 111.76) (end 118.11 100.33) (width 1) (layer "B.Cu") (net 3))
 (segment (start 113.92 90.45) (end 113.82 90.55) (width 1) (layer "B.Cu") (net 1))
 (segment (start 118.11 90.45) (end 113.92 90.45) (width 1) (layer "B.Cu") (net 1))
 (segment (start 121.64 90.45) (end 121.92 90.17) (width 1) (layer "B.Cu") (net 1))
 (segment (start 118.11 90.45) (end 121.64 90.45) (width 1) (layer "B.Cu") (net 1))
 (segment (start 102.87 100.33) (end 103.25 99.95) (width 1) (layer "B.Cu") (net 5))
 (segment (start 102.87 111.76) (end 102.87 100.33) (width 1) (layer "B.Cu") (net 5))
 (segment (start 104.14 99.06) (end 104.14 96.8) (width 1) (layer "B.Cu") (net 5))
 (segment (start 103.25 99.95) (end 104.14 99.06) (width 1) (layer "B.Cu") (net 5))
 (segment (start 98.82 99.95) (end 103.25 99.95) (width 1) (layer "B.Cu") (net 5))
 (segment (start 98.92 90.45) (end 98.82 90.55) (width 1) (layer "B.Cu") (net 8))
 (segment (start 102.87 90.45) (end 106.4 90.45) (width 1) (layer "B.Cu") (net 8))
 (segment (start 106.4 90.45) (end 106.68 90.17) (width 1) (layer "B.Cu") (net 8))
 (segment (start 102.87 90.45) (end 98.92 90.45) (width 1) (layer "B.Cu") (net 8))
 (segment (start 83.82 99.95) (end 88.01 99.95) (width 1) (layer "B.Cu") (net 7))
 (segment (start 88.01 99.95) (end 88.9 99.06) (width 1) (layer "B.Cu") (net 7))
 (segment (start 87.63 100.33) (end 88.01 99.95) (width 1) (layer "B.Cu") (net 7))
 (segment (start 87.63 111.76) (end 87.63 100.33) (width 1) (layer "B.Cu") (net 7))
 (segment (start 88.9 99.06) (end 88.9 96.8) (width 1) (layer "B.Cu") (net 7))
 (segment (start 87.63 90.55) (end 83.82 90.55) (width 1) (layer "B.Cu") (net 6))
 (segment (start 91.16 90.45) (end 91.44 90.17) (width 1) (layer "B.Cu") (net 6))
 (segment (start 87.63 90.45) (end 91.16 90.45) (width 1) (layer "B.Cu") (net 6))
 (segment (start 119.38 93.7) (end 122.2 93.7) (width 1) (layer "B.Cu") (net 4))
 (segment (start 93.98 92.71) (end 93.98 87.35) (width 1) (layer "B.Cu") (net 4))
 (segment (start 87.63 87.35) (end 80.29 87.35) (width 1) (layer "B.Cu") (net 4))
 (segment (start 80.01 109.22) (end 80.01 111.76) (width 1) (layer "B.Cu") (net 4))
 (segment (start 92.99 93.7) (end 93.98 92.71) (width 1) (layer "B.Cu") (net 4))
 (segment (start 124.46 91.44) (end 124.46 88.9) (width 1) (layer "B.Cu") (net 4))
 (segment (start 108.23 93.7) (end 109.22 92.71) (width 1) (layer "B.Cu") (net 4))
 (segment (start 78.61 89.03) (end 78.61 107.82) (width 1) (layer "B.Cu") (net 4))
 (segment (start 122.91 87.35) (end 124.46 88.9) (width 1) (layer "B.Cu") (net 4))
 (segment (start 88.9 93.7) (end 92.99 93.7) (width 1) (layer "B.Cu") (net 4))
 (segment (start 109.22 92.71) (end 109.22 87.35) (width 1) (layer "B.Cu") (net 4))
 (segment (start 87.63 87.35) (end 122.91 87.35) (width 1) (layer "B.Cu") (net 4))
 (segment (start 122.2 93.7) (end 124.46 91.44) (width 1) (layer "B.Cu") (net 4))
 (segment (start 78.61 107.82) (end 80.01 109.22) (width 1) (layer "B.Cu") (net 4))
 (segment (start 80.29 87.35) (end 78.61 89.03) (width 1) (layer "B.Cu") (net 4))
 (segment (start 104.14 93.7) (end 108.23 93.7) (width 1) (layer "B.Cu") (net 4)))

